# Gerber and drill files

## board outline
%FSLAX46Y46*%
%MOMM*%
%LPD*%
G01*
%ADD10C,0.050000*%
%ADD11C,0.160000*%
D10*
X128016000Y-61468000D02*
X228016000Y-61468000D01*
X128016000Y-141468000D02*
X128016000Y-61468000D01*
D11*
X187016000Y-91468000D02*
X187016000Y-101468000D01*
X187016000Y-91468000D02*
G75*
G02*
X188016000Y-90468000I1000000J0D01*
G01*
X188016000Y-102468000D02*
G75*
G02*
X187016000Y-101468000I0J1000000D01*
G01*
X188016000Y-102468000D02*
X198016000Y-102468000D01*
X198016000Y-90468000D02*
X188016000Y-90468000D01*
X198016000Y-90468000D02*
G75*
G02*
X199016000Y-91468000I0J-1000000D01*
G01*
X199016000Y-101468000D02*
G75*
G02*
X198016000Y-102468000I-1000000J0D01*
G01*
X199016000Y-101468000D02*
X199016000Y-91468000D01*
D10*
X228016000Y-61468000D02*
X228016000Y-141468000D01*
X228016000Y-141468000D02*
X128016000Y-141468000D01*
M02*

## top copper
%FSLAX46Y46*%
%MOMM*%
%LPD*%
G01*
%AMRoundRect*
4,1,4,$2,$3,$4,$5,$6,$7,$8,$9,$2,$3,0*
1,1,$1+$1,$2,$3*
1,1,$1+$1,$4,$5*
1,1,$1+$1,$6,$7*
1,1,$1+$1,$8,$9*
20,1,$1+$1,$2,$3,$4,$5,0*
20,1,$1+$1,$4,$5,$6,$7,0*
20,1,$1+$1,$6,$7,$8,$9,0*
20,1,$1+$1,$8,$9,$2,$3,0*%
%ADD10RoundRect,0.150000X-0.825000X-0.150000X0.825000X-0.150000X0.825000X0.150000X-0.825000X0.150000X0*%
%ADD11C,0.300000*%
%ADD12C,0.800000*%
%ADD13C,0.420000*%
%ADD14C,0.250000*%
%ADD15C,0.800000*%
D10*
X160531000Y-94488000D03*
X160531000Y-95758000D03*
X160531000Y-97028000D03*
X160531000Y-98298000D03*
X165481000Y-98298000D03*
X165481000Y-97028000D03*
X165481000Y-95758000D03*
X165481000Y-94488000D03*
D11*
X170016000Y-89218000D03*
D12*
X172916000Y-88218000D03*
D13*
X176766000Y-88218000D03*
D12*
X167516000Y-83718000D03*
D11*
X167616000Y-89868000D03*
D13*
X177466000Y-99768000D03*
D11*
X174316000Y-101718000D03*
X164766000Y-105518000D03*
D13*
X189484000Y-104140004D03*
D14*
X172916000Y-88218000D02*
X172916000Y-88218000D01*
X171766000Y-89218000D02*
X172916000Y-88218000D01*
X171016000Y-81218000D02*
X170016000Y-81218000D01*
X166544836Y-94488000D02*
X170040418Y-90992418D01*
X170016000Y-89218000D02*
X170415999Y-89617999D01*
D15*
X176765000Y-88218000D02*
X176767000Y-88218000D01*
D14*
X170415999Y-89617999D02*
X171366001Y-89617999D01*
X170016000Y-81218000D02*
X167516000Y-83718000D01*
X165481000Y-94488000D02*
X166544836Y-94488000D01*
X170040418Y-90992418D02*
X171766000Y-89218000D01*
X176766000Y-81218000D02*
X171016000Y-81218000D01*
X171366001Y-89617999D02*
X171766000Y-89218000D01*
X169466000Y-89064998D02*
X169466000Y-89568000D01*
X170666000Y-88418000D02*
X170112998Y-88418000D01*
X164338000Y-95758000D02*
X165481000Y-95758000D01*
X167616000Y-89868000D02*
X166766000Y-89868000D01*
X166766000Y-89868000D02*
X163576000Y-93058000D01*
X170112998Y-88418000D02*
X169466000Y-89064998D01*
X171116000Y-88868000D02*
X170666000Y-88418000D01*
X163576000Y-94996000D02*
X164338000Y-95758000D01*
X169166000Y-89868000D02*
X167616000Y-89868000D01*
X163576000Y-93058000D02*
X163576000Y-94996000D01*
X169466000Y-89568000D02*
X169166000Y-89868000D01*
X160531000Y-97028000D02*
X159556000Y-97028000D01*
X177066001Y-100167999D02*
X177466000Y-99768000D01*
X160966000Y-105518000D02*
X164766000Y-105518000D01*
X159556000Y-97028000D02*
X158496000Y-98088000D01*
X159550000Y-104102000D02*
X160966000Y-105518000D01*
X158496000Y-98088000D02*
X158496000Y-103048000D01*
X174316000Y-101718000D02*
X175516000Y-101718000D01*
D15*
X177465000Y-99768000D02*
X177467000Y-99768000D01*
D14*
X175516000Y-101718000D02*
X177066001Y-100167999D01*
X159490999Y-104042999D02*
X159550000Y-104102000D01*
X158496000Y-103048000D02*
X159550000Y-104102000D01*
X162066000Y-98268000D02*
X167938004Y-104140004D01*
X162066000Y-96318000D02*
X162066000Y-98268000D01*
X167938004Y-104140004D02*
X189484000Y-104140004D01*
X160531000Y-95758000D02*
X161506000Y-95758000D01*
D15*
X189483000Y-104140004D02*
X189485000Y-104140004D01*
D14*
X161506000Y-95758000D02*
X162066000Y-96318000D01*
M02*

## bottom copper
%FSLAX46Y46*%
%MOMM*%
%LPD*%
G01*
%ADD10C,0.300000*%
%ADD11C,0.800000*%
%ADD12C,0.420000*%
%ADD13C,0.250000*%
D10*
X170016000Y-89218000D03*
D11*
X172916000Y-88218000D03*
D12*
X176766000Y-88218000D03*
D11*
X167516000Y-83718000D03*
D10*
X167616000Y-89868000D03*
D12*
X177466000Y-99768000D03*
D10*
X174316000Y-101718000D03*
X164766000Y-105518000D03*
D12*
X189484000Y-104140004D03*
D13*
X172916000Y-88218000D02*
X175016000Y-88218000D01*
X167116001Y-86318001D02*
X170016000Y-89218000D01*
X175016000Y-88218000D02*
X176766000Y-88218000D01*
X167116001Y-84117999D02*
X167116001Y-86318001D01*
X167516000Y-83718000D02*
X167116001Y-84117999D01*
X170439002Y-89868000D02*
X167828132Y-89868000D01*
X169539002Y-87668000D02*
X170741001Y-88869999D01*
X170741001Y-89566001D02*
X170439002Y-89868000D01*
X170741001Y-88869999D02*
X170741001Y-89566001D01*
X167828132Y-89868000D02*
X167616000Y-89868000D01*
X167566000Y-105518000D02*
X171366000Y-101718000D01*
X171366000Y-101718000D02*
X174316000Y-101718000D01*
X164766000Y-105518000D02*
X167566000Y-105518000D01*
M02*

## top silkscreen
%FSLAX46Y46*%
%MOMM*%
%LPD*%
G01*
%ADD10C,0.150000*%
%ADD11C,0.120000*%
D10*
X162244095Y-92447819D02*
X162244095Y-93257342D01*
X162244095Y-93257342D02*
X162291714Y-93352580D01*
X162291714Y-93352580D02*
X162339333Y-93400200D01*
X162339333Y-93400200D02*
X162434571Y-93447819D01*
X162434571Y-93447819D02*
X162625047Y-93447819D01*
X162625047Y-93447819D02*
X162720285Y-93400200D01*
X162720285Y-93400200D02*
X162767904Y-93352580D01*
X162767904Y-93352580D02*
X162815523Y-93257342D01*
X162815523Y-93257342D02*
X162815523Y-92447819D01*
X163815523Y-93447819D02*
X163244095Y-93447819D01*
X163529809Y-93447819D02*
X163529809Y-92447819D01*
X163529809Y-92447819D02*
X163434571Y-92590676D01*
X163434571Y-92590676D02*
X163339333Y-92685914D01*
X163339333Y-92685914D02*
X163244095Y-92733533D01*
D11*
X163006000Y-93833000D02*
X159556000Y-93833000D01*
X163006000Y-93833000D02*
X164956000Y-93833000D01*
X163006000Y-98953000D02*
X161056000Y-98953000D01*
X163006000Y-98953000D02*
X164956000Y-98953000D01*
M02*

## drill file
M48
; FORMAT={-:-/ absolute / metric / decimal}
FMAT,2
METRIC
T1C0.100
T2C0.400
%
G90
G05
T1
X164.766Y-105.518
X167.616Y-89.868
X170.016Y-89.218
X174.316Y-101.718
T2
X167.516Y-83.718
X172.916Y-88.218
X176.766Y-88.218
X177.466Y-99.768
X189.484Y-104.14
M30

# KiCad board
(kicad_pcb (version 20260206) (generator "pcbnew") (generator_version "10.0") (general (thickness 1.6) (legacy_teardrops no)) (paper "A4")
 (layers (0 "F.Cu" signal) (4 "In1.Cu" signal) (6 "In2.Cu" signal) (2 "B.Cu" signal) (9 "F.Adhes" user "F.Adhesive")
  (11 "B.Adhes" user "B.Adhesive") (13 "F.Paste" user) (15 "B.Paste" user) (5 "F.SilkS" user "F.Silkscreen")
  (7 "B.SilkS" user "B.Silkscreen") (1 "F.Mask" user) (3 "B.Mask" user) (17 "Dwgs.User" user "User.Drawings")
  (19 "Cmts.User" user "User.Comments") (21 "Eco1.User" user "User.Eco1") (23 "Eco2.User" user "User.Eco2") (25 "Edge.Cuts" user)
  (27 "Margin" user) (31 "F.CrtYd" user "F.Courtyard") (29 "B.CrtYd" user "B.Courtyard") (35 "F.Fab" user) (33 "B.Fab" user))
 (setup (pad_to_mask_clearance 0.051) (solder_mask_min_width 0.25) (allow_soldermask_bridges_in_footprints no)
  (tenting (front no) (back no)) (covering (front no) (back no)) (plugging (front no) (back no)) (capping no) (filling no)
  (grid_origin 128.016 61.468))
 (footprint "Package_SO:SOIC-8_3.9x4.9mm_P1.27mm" (layer "F.Cu") (at 163.006 96.393)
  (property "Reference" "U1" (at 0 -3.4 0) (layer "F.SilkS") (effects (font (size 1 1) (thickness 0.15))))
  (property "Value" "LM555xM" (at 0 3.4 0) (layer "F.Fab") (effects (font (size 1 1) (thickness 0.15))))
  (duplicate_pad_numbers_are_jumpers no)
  (fp_line (start 0 -2.56) (end -3.45 -2.56) (stroke (width 0.12) (type solid)) (layer "F.SilkS"))
  (fp_line (start 0 -2.56) (end 1.95 -2.56) (stroke (width 0.12) (type solid)) (layer "F.SilkS"))
  (fp_line (start 0 2.56) (end -1.95 2.56) (stroke (width 0.12) (type solid)) (layer "F.SilkS"))
  (fp_line (start 0 2.56) (end 1.95 2.56) (stroke (width 0.12) (type solid)) (layer "F.SilkS"))
  (pad "1" smd roundrect (at -2.475 -1.905) (size 1.95 0.6) (layers "F.Cu" "F.Mask" "F.Paste") (roundrect_rratio 0.25) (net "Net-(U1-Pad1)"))
  (pad "2" smd roundrect (at -2.475 -0.635) (size 1.95 0.6) (layers "F.Cu" "F.Mask" "F.Paste") (roundrect_rratio 0.25) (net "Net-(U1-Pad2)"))
  (pad "3" smd roundrect (at -2.475 0.635) (size 1.95 0.6) (layers "F.Cu" "F.Mask" "F.Paste") (roundrect_rratio 0.25) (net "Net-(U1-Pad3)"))
  (pad "4" smd roundrect (at -2.475 1.905) (size 1.95 0.6) (layers "F.Cu" "F.Mask" "F.Paste") (roundrect_rratio 0.25) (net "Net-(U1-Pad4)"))
  (pad "5" smd roundrect (at 2.475 1.905) (size 1.95 0.6) (layers "F.Cu" "F.Mask" "F.Paste") (roundrect_rratio 0.25) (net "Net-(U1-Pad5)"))
  (pad "6" smd roundrect (at 2.475 0.635) (size 1.95 0.6) (layers "F.Cu" "F.Mask" "F.Paste") (roundrect_rratio 0.25) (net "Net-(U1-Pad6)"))
  (pad "7" smd roundrect (at 2.475 -0.635) (size 1.95 0.6) (layers "F.Cu" "F.Mask" "F.Paste") (roundrect_rratio 0.25) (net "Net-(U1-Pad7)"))
  (pad "8" smd roundrect (at 2.475 -1.905) (size 1.95 0.6) (layers "F.Cu" "F.Mask" "F.Paste") (roundrect_rratio 0.25) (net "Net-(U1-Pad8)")))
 (gr_line (start 128.016 61.468) (end 228.016 61.468) (stroke (width 0.05) (type solid)) (layer "Edge.Cuts"))
 (gr_line (start 128.016 141.468) (end 128.016 61.468) (stroke (width 0.05) (type solid)) (layer "Edge.Cuts"))
 (gr_line (start 187.016 91.468) (end 187.016 101.468) (stroke (width 0.16) (type solid)) (layer "Edge.Cuts"))
 (gr_arc (start 187.016 91.468) (mid 187.308893 90.760893) (end 188.016 90.468) (stroke (width 0.16) (type solid)) (layer "Edge.Cuts"))
 (gr_arc (start 188.016 102.468) (mid 187.308893 102.175107) (end 187.016 101.468) (stroke (width 0.16) (type solid)) (layer "Edge.Cuts"))
 (gr_line (start 188.016 102.468) (end 198.016 102.468) (stroke (width 0.16) (type solid)) (layer "Edge.Cuts"))
 (gr_line (start 198.016 90.468) (end 188.016 90.468) (stroke (width 0.16) (type solid)) (layer "Edge.Cuts"))
 (gr_arc (start 198.016 90.468) (mid 198.723107 90.760893) (end 199.016 91.468) (stroke (width 0.16) (type solid)) (layer "Edge.Cuts"))
 (gr_arc (start 199.016 101.468) (mid 198.723107 102.175107) (end 198.016 102.468) (stroke (width 0.16) (type solid)) (layer "Edge.Cuts"))
 (gr_line (start 199.016 101.468) (end 199.016 91.468) (stroke (width 0.16) (type solid)) (layer "Edge.Cuts"))
 (gr_line (start 228.016 61.468) (end 228.016 141.468) (stroke (width 0.05) (type solid)) (layer "Edge.Cuts"))
 (gr_line (start 228.016 141.468) (end 128.016 141.468) (stroke (width 0.05) (type solid)) (layer "Edge.Cuts"))
 (segment (start 172.916 88.218) (end 172.916 88.218) (width 0.25) (layer "F.Cu") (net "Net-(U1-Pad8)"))
 (segment (start 171.766 89.218) (end 172.916 88.218) (width 0.25) (layer "F.Cu") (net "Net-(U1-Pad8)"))
 (segment (start 171.016 81.218) (end 170.016 81.218) (width 0.25) (layer "F.Cu") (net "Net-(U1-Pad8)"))
 (segment (start 166.544836 94.488) (end 170.040418 90.992418) (width 0.25) (layer "F.Cu") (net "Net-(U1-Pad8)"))
 (segment (start 170.016 89.218) (end 170.415999 89.617999) (width 0.25) (layer "F.Cu") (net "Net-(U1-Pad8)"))
 (segment (start 176.765 88.218) (end 176.767 88.218) (width 0.8) (layer "F.Cu") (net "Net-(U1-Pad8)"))
 (segment (start 170.415999 89.617999) (end 171.366001 89.617999) (width 0.25) (layer "F.Cu") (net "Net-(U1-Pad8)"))
 (segment (start 170.016 81.218) (end 167.516 83.718) (width 0.25) (layer "F.Cu") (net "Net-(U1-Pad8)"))
 (segment (start 165.481 94.488) (end 166.544836 94.488) (width 0.25) (layer "F.Cu") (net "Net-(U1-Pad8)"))
 (segment (start 170.040418 90.992418) (end 171.766 89.218) (width 0.25) (layer "F.Cu") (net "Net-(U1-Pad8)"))
 (segment (start 176.766 81.218) (end 171.016 81.218) (width 0.25) (layer "F.Cu") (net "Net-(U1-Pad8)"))
 (segment (start 171.366001 89.617999) (end 171.766 89.218) (width 0.25) (layer "F.Cu") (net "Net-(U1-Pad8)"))
 (via (at 170.016 89.218) (size 0.3) (drill 0.1) (layers "F.Cu" "B.Cu") (capping no) (covering (front no) (back no))
  (plugging (front no) (back no)) (filling no) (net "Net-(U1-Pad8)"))
 (via (at 172.916 88.218) (size 0.8) (drill 0.4) (layers "F.Cu" "B.Cu") (capping no) (covering (front no) (back no))
  (plugging (front no) (back no)) (filling no) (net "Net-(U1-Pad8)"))
 (via (at 176.766 88.218) (size 0.42) (drill 0.4) (layers "F.Cu" "B.Cu") (capping no) (covering (front no) (back no))
  (plugging (front no) (back no)) (filling no) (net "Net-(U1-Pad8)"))
 (via (at 167.516 83.718) (size 0.8) (drill 0.4) (layers "F.Cu" "B.Cu") (capping no) (covering (front no) (back no))
  (plugging (front no) (back no)) (filling no) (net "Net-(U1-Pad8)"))
 (segment (start 172.916 88.218) (end 175.016 88.218) (width 0.25) (layer "B.Cu") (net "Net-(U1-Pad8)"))
 (segment (start 167.116001 86.318001) (end 170.016 89.218) (width 0.25) (layer "B.Cu") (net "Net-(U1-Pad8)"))
 (segment (start 175.016 88.218) (end 176.766 88.218) (width 0.25) (layer "B.Cu") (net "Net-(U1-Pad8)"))
 (segment (start 167.116001 84.117999) (end 167.116001 86.318001) (width 0.25) (layer "B.Cu") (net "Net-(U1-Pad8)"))
 (segment (start 167.516 83.718) (end 167.116001 84.117999) (width 0.25) (layer "B.Cu") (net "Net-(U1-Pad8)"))
 (segment (start 169.466 89.064998) (end 169.466 89.568) (width 0.25) (layer "F.Cu") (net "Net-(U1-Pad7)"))
 (segment (start 170.666 88.418) (end 170.112998 88.418) (width 0.25) (layer "F.Cu") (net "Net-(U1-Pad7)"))
 (segment (start 164.338 95.758) (end 165.481 95.758) (width 0.25) (layer "F.Cu") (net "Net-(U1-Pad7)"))
 (segment (start 167.616 89.868) (end 166.766 89.868) (width 0.25) (layer "F.Cu") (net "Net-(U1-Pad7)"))
 (segment (start 166.766 89.868) (end 163.576 93.058) (width 0.25) (layer "F.Cu") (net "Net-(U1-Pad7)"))
 (segment (start 170.112998 88.418) (end 169.466 89.064998) (width 0.25) (layer "F.Cu") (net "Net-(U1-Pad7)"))
 (segment (start 171.116 88.868) (end 170.666 88.418) (width 0.25) (layer "F.Cu") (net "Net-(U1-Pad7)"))
 (segment (start 163.576 94.996) (end 164.338 95.758) (width 0.25) (layer "F.Cu") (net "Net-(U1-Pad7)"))
 (segment (start 169.166 89.868) (end 167.616 89.868) (width 0.25) (layer "F.Cu") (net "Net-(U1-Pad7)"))
 (segment (start 163.576 93.058) (end 163.576 94.996) (width 0.25) (layer "F.Cu") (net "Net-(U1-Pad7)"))
 (segment (start 169.466 89.568) (end 169.166 89.868) (width 0.25) (layer "F.Cu") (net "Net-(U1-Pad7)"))
 (via (at 167.616 89.868) (size 0.3) (drill 0.1) (layers "F.Cu" "B.Cu") (capping no) (covering (front no) (back no))
  (plugging (front no) (back no)) (filling no) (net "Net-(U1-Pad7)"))
 (segment (start 170.439002 89.868) (end 167.828132 89.868) (width 0.25) (layer "B.Cu") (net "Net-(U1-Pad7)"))
 (segment (start 169.539002 87.668) (end 170.741001 88.869999) (width 0.25) (layer "B.Cu") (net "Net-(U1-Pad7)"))
 (segment (start 170.741001 89.566001) (end 170.439002 89.868) (width 0.25) (layer "B.Cu") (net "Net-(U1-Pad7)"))
 (segment (start 170.741001 88.869999) (end 170.741001 89.566001) (width 0.25) (layer "B.Cu") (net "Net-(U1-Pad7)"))
 (segment (start 167.828132 89.868) (end 167.616 89.868) (width 0.25) (layer "B.Cu") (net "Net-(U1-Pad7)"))
 (segment (start 160.531 97.028) (end 159.556 97.028) (width 0.25) (layer "F.Cu") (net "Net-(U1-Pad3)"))
 (segment (start 177.066001 100.167999) (end 177.466 99.768) (width 0.25) (layer "F.Cu") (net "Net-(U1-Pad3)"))
 (segment (start 160.966 105.518) (end 164.766 105.518) (width 0.25) (layer "F.Cu") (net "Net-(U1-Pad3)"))
 (segment (start 159.556 97.028) (end 158.496 98.088) (width 0.25) (layer "F.Cu") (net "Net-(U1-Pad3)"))
 (segment (start 159.55 104.102) (end 160.966 105.518) (width 0.25) (layer "F.Cu") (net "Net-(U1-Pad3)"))
 (segment (start 158.496 98.088) (end 158.496 103.048) (width 0.25) (layer "F.Cu") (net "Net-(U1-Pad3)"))
 (segment (start 174.316 101.718) (end 175.516 101.718) (width 0.25) (layer "F.Cu") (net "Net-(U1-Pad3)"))
 (segment (start 177.465 99.768) (end 177.467 99.768) (width 0.8) (layer "F.Cu") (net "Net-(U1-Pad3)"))
 (segment (start 175.516 101.718) (end 177.066001 100.167999) (width 0.25) (layer "F.Cu") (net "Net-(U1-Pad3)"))
 (segment (start 159.490999 104.042999) (end 159.55 104.102) (width 0.25) (layer "F.Cu") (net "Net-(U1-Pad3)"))
 (segment (start 158.496 103.048) (end 159.55 104.102) (width 0.25) (layer "F.Cu") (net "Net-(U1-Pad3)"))
 (via (at 177.466 99.768) (size 0.42) (drill 0.4) (layers "F.Cu" "B.Cu") (capping no) (covering (front no) (back no))
  (plugging (front no) (back no)) (filling no) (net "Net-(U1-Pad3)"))
 (via (at 174.316 101.718) (size 0.3) (drill 0.1) (layers "F.Cu" "B.Cu") (capping no) (covering (front no) (back no))
  (plugging (front no) (back no)) (filling no) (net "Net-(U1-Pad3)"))
 (via (at 164.766 105.518) (size 0.3) (drill 0.1) (layers "F.Cu" "B.Cu") (capping no) (covering (front no) (back no))
  (plugging (front no) (back no)) (filling no) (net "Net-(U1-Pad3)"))
 (segment (start 167.566 105.518) (end 171.366 101.718) (width 0.25) (layer "B.Cu") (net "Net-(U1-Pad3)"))
 (segment (start 171.366 101.718) (end 174.316 101.718) (width 0.25) (layer "B.Cu") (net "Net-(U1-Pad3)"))
 (segment (start 164.766 105.518) (end 167.566 105.518) (width 0.25) (layer "B.Cu") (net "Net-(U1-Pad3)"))
 (segment (start 162.066 98.268) (end 167.938004 104.140004) (width 0.25) (layer "F.Cu") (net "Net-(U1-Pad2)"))
 (segment (start 162.066 96.318) (end 162.066 98.268) (width 0.25) (layer "F.Cu") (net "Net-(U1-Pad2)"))
 (segment (start 167.938004 104.140004) (end 189.484 104.140004) (width 0.25) (layer "F.Cu") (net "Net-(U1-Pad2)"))
 (segment (start 160.531 95.758) (end 161.506 95.758) (width 0.25) (layer "F.Cu") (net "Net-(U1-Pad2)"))
 (segment (start 189.483 104.140004) (end 189.485 104.140004) (width 0.8) (layer "F.Cu") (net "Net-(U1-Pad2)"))
 (segment (start 161.506 95.758) (end 162.066 96.318) (width 0.25) (layer "F.Cu") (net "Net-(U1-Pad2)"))
 (via (at 189.484 104.140004) (size 0.42) (drill 0.4) (layers "F.Cu" "B.Cu") (capping no) (covering (front no) (back no))
  (plugging (front no) (back no)) (filling no) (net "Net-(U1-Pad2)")))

